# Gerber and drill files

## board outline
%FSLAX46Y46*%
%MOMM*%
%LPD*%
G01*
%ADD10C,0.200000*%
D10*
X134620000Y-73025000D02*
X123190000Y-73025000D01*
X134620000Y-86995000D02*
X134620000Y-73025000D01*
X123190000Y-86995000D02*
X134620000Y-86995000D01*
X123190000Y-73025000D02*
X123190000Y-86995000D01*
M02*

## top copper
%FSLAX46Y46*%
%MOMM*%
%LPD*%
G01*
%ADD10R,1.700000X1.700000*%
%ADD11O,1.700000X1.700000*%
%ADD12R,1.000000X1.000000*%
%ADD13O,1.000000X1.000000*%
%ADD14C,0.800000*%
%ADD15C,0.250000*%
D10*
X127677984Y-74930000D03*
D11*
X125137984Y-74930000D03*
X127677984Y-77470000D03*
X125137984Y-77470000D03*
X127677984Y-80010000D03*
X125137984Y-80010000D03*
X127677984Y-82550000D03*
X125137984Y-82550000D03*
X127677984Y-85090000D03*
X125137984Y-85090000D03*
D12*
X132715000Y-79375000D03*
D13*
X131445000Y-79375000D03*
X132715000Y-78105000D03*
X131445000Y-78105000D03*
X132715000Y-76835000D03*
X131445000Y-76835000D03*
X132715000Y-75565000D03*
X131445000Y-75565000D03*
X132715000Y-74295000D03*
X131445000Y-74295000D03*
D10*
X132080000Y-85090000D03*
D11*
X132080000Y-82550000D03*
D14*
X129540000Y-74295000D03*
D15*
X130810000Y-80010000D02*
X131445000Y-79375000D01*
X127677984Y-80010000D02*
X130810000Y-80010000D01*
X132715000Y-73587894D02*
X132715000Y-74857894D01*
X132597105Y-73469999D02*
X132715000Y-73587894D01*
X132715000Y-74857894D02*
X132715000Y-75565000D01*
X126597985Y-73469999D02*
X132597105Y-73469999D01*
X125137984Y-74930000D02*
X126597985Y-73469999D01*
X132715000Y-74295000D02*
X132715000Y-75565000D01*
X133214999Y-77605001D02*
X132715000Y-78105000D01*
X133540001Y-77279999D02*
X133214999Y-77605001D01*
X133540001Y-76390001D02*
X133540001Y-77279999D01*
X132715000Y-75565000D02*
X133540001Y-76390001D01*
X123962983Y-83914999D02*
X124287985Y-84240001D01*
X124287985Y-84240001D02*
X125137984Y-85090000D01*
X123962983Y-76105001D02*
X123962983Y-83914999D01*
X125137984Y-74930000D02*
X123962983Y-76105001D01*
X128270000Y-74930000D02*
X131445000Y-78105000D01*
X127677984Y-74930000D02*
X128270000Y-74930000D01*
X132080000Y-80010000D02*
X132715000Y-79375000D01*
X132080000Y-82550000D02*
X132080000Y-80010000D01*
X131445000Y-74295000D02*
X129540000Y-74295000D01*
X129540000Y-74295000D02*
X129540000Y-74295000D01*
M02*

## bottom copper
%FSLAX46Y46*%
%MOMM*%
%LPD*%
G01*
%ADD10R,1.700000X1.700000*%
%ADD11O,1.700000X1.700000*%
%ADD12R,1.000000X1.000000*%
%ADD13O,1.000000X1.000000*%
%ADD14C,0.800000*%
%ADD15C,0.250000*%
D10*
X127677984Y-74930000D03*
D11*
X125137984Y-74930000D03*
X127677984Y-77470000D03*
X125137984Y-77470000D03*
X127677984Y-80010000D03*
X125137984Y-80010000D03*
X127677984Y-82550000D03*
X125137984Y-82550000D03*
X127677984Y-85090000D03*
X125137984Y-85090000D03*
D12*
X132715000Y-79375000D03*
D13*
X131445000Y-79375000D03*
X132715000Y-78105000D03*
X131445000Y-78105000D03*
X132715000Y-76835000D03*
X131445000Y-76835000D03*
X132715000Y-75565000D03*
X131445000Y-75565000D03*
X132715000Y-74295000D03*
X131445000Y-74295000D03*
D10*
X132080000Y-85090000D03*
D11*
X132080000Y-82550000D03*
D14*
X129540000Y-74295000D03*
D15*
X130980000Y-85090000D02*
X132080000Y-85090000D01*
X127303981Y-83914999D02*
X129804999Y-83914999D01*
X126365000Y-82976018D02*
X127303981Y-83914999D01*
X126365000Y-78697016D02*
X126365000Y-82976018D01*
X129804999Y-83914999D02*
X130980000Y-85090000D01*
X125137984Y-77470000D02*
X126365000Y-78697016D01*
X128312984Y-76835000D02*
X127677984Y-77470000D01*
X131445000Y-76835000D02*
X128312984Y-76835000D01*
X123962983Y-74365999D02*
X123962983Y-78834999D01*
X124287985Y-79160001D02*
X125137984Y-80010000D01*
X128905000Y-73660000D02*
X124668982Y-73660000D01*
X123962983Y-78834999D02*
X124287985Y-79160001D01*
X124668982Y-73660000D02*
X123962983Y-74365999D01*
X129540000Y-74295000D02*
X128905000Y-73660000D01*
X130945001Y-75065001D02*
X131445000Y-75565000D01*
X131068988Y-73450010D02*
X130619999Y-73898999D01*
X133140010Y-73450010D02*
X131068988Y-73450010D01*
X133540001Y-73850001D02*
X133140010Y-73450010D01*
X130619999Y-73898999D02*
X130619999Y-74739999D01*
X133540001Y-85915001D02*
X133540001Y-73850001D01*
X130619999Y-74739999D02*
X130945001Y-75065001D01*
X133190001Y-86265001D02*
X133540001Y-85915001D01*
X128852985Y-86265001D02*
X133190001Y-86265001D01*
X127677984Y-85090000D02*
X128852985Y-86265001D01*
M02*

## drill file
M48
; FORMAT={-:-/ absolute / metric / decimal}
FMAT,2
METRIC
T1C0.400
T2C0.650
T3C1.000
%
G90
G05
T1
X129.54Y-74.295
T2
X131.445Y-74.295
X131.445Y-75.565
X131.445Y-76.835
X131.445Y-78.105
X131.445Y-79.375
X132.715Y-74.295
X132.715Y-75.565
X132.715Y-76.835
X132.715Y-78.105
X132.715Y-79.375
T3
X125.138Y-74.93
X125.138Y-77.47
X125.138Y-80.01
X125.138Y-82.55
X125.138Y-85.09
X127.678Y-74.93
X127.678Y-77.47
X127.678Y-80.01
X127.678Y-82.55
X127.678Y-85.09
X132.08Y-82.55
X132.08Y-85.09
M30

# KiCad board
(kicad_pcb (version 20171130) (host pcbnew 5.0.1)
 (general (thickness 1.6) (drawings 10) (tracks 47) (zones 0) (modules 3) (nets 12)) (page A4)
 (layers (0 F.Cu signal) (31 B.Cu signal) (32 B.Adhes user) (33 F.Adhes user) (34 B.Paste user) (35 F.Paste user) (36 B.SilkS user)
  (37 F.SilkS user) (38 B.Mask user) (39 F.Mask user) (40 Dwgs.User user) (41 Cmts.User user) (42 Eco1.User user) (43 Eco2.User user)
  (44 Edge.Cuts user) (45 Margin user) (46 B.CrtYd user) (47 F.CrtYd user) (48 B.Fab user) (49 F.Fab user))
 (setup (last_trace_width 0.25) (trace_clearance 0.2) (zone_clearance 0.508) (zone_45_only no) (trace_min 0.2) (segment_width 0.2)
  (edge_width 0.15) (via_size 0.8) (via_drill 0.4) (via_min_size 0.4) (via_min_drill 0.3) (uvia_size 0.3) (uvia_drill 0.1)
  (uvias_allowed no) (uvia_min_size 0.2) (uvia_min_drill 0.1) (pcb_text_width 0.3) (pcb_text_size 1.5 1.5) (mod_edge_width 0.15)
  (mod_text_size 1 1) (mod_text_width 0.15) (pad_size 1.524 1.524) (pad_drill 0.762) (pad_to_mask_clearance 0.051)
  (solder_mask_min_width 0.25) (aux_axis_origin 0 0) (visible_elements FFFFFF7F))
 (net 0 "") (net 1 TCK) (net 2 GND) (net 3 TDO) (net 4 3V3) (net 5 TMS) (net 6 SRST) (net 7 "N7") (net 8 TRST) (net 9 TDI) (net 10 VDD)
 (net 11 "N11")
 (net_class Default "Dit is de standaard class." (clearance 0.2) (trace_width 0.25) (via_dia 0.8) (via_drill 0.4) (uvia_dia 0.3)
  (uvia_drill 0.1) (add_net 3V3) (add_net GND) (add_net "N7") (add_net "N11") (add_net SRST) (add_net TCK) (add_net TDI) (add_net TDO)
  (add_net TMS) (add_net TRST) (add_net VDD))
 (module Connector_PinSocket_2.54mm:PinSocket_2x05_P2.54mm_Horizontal (layer F.Cu) (at 127.677984 74.93)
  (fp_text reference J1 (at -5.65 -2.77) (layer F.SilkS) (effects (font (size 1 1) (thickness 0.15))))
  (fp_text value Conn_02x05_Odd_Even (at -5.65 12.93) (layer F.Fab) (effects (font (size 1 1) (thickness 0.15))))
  (pad 1 thru_hole rect (at 0 0) (size 1.7 1.7) (drill 1) (layers *.Cu *.Mask) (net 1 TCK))
  (pad 2 thru_hole oval (at -2.54 0) (size 1.7 1.7) (drill 1) (layers *.Cu *.Mask) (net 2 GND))
  (pad 3 thru_hole oval (at 0 2.54) (size 1.7 1.7) (drill 1) (layers *.Cu *.Mask) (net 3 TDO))
  (pad 4 thru_hole oval (at -2.54 2.54) (size 1.7 1.7) (drill 1) (layers *.Cu *.Mask) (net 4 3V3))
  (pad 5 thru_hole oval (at 0 5.08) (size 1.7 1.7) (drill 1) (layers *.Cu *.Mask) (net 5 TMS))
  (pad 6 thru_hole oval (at -2.54 5.08) (size 1.7 1.7) (drill 1) (layers *.Cu *.Mask) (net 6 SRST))
  (pad 7 thru_hole oval (at 0 7.62) (size 1.7 1.7) (drill 1) (layers *.Cu *.Mask) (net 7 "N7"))
  (pad 8 thru_hole oval (at -2.54 7.62) (size 1.7 1.7) (drill 1) (layers *.Cu *.Mask) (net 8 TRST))
  (pad 9 thru_hole oval (at 0 10.16) (size 1.7 1.7) (drill 1) (layers *.Cu *.Mask) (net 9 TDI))
  (pad 10 thru_hole oval (at -2.54 10.16) (size 1.7 1.7) (drill 1) (layers *.Cu *.Mask) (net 2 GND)))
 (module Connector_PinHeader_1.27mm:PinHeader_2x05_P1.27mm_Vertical (layer F.Cu) (at 132.715 79.375 180)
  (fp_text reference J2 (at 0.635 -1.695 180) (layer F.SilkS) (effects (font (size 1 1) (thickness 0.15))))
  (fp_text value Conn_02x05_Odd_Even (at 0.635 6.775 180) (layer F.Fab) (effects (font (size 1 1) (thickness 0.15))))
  (pad 1 thru_hole rect (at 0 0 180) (size 1 1) (drill 0.65) (layers *.Cu *.Mask) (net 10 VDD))
  (pad 2 thru_hole oval (at 1.27 0 180) (size 1 1) (drill 0.65) (layers *.Cu *.Mask) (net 5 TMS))
  (pad 3 thru_hole oval (at 0 1.27 180) (size 1 1) (drill 0.65) (layers *.Cu *.Mask) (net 2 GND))
  (pad 4 thru_hole oval (at 1.27 1.27 180) (size 1 1) (drill 0.65) (layers *.Cu *.Mask) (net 1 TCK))
  (pad 5 thru_hole oval (at 0 2.54 180) (size 1 1) (drill 0.65) (layers *.Cu *.Mask) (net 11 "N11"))
  (pad 6 thru_hole oval (at 1.27 2.54 180) (size 1 1) (drill 0.65) (layers *.Cu *.Mask) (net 3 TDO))
  (pad 7 thru_hole oval (at 0 3.81 180) (size 1 1) (drill 0.65) (layers *.Cu *.Mask) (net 2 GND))
  (pad 8 thru_hole oval (at 1.27 3.81 180) (size 1 1) (drill 0.65) (layers *.Cu *.Mask) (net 9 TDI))
  (pad 9 thru_hole oval (at 0 5.08 180) (size 1 1) (drill 0.65) (layers *.Cu *.Mask) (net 2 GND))
  (pad 10 thru_hole oval (at 1.27 5.08 180) (size 1 1) (drill 0.65) (layers *.Cu *.Mask) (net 6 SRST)))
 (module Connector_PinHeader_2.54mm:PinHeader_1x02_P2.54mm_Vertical (layer F.Cu) (at 132.08 85.09 180)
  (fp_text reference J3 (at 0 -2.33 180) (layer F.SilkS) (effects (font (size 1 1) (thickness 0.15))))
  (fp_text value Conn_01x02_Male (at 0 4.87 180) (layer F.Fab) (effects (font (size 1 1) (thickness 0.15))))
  (pad 1 thru_hole rect (at 0 0 180) (size 1.7 1.7) (drill 1) (layers *.Cu *.Mask) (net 4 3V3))
  (pad 2 thru_hole oval (at 0 2.54 180) (size 1.7 1.7) (drill 1) (layers *.Cu *.Mask) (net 10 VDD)))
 (gr_line (start 134.62 73.025) (end 123.19 73.025) (layer Edge.Cuts) (width 0.2))
 (gr_line (start 134.62 86.995) (end 134.62 73.025) (layer Edge.Cuts) (width 0.2))
 (gr_line (start 123.19 86.995) (end 134.62 86.995) (layer Edge.Cuts) (width 0.2))
 (gr_line (start 123.19 73.025) (end 123.19 86.995) (layer Edge.Cuts) (width 0.2))
 (segment (start 130.81 80.01) (end 131.445 79.375) (width 0.25) (layer F.Cu) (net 5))
 (segment (start 127.677984 80.01) (end 130.81 80.01) (width 0.25) (layer F.Cu) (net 5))
 (segment (start 132.715 73.587894) (end 132.715 74.857894) (width 0.25) (layer F.Cu) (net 2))
 (segment (start 132.597105 73.469999) (end 132.715 73.587894) (width 0.25) (layer F.Cu) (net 2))
 (segment (start 132.715 74.857894) (end 132.715 75.565) (width 0.25) (layer F.Cu) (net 2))
 (segment (start 126.597985 73.469999) (end 132.597105 73.469999) (width 0.25) (layer F.Cu) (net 2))
 (segment (start 125.137984 74.93) (end 126.597985 73.469999) (width 0.25) (layer F.Cu) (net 2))
 (segment (start 132.715 74.295) (end 132.715 75.565) (width 0.25) (layer F.Cu) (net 2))
 (segment (start 133.214999 77.605001) (end 132.715 78.105) (width 0.25) (layer F.Cu) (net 2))
 (segment (start 133.540001 77.279999) (end 133.214999 77.605001) (width 0.25) (layer F.Cu) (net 2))
 (segment (start 133.540001 76.390001) (end 133.540001 77.279999) (width 0.25) (layer F.Cu) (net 2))
 (segment (start 132.715 75.565) (end 133.540001 76.390001) (width 0.25) (layer F.Cu) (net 2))
 (segment (start 123.962983 83.914999) (end 124.287985 84.240001) (width 0.25) (layer F.Cu) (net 2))
 (segment (start 124.287985 84.240001) (end 125.137984 85.09) (width 0.25) (layer F.Cu) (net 2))
 (segment (start 123.962983 76.105001) (end 123.962983 83.914999) (width 0.25) (layer F.Cu) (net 2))
 (segment (start 125.137984 74.93) (end 123.962983 76.105001) (width 0.25) (layer F.Cu) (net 2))
 (segment (start 128.27 74.93) (end 131.445 78.105) (width 0.25) (layer F.Cu) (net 1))
 (segment (start 127.677984 74.93) (end 128.27 74.93) (width 0.25) (layer F.Cu) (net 1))
 (segment (start 130.98 85.09) (end 132.08 85.09) (width 0.25) (layer B.Cu) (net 4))
 (segment (start 127.303981 83.914999) (end 129.804999 83.914999) (width 0.25) (layer B.Cu) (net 4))
 (segment (start 126.365 82.976018) (end 127.303981 83.914999) (width 0.25) (layer B.Cu) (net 4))
 (segment (start 126.365 78.697016) (end 126.365 82.976018) (width 0.25) (layer B.Cu) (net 4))
 (segment (start 129.804999 83.914999) (end 130.98 85.09) (width 0.25) (layer B.Cu) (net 4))
 (segment (start 125.137984 77.47) (end 126.365 78.697016) (width 0.25) (layer B.Cu) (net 4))
 (segment (start 132.08 80.01) (end 132.715 79.375) (width 0.25) (layer F.Cu) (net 10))
 (segment (start 132.08 82.55) (end 132.08 80.01) (width 0.25) (layer F.Cu) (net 10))
 (segment (start 128.312984 76.835) (end 127.677984 77.47) (width 0.25) (layer B.Cu) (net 3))
 (segment (start 131.445 76.835) (end 128.312984 76.835) (width 0.25) (layer B.Cu) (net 3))
 (segment (start 131.445 74.295) (end 129.54 74.295) (width 0.25) (layer F.Cu) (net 6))
 (segment (start 129.54 74.295) (end 129.54 74.295) (width 0.25) (layer F.Cu) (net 6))
 (via (at 129.54 74.295) (size 0.8) (drill 0.4) (layers F.Cu B.Cu) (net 6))
 (segment (start 123.962983 74.365999) (end 123.962983 78.834999) (width 0.25) (layer B.Cu) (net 6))
 (segment (start 124.287985 79.160001) (end 125.137984 80.01) (width 0.25) (layer B.Cu) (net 6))
 (segment (start 128.905 73.66) (end 124.668982 73.66) (width 0.25) (layer B.Cu) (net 6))
 (segment (start 123.962983 78.834999) (end 124.287985 79.160001) (width 0.25) (layer B.Cu) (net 6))
 (segment (start 124.668982 73.66) (end 123.962983 74.365999) (width 0.25) (layer B.Cu) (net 6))
 (segment (start 129.54 74.295) (end 128.905 73.66) (width 0.25) (layer B.Cu) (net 6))
 (segment (start 130.945001 75.065001) (end 131.445 75.565) (width 0.25) (layer B.Cu) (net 9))
 (segment (start 131.068988 73.45001) (end 130.619999 73.898999) (width 0.25) (layer B.Cu) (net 9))
 (segment (start 133.14001 73.45001) (end 131.068988 73.45001) (width 0.25) (layer B.Cu) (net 9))
 (segment (start 133.540001 73.850001) (end 133.14001 73.45001) (width 0.25) (layer B.Cu) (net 9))
 (segment (start 130.619999 73.898999) (end 130.619999 74.739999) (width 0.25) (layer B.Cu) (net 9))
 (segment (start 133.540001 85.915001) (end 133.540001 73.850001) (width 0.25) (layer B.Cu) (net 9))
 (segment (start 130.619999 74.739999) (end 130.945001 75.065001) (width 0.25) (layer B.Cu) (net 9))
 (segment (start 133.190001 86.265001) (end 133.540001 85.915001) (width 0.25) (layer B.Cu) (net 9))
 (segment (start 128.852985 86.265001) (end 133.190001 86.265001) (width 0.25) (layer B.Cu) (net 9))
 (segment (start 127.677984 85.09) (end 128.852985 86.265001) (width 0.25) (layer B.Cu) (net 9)))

